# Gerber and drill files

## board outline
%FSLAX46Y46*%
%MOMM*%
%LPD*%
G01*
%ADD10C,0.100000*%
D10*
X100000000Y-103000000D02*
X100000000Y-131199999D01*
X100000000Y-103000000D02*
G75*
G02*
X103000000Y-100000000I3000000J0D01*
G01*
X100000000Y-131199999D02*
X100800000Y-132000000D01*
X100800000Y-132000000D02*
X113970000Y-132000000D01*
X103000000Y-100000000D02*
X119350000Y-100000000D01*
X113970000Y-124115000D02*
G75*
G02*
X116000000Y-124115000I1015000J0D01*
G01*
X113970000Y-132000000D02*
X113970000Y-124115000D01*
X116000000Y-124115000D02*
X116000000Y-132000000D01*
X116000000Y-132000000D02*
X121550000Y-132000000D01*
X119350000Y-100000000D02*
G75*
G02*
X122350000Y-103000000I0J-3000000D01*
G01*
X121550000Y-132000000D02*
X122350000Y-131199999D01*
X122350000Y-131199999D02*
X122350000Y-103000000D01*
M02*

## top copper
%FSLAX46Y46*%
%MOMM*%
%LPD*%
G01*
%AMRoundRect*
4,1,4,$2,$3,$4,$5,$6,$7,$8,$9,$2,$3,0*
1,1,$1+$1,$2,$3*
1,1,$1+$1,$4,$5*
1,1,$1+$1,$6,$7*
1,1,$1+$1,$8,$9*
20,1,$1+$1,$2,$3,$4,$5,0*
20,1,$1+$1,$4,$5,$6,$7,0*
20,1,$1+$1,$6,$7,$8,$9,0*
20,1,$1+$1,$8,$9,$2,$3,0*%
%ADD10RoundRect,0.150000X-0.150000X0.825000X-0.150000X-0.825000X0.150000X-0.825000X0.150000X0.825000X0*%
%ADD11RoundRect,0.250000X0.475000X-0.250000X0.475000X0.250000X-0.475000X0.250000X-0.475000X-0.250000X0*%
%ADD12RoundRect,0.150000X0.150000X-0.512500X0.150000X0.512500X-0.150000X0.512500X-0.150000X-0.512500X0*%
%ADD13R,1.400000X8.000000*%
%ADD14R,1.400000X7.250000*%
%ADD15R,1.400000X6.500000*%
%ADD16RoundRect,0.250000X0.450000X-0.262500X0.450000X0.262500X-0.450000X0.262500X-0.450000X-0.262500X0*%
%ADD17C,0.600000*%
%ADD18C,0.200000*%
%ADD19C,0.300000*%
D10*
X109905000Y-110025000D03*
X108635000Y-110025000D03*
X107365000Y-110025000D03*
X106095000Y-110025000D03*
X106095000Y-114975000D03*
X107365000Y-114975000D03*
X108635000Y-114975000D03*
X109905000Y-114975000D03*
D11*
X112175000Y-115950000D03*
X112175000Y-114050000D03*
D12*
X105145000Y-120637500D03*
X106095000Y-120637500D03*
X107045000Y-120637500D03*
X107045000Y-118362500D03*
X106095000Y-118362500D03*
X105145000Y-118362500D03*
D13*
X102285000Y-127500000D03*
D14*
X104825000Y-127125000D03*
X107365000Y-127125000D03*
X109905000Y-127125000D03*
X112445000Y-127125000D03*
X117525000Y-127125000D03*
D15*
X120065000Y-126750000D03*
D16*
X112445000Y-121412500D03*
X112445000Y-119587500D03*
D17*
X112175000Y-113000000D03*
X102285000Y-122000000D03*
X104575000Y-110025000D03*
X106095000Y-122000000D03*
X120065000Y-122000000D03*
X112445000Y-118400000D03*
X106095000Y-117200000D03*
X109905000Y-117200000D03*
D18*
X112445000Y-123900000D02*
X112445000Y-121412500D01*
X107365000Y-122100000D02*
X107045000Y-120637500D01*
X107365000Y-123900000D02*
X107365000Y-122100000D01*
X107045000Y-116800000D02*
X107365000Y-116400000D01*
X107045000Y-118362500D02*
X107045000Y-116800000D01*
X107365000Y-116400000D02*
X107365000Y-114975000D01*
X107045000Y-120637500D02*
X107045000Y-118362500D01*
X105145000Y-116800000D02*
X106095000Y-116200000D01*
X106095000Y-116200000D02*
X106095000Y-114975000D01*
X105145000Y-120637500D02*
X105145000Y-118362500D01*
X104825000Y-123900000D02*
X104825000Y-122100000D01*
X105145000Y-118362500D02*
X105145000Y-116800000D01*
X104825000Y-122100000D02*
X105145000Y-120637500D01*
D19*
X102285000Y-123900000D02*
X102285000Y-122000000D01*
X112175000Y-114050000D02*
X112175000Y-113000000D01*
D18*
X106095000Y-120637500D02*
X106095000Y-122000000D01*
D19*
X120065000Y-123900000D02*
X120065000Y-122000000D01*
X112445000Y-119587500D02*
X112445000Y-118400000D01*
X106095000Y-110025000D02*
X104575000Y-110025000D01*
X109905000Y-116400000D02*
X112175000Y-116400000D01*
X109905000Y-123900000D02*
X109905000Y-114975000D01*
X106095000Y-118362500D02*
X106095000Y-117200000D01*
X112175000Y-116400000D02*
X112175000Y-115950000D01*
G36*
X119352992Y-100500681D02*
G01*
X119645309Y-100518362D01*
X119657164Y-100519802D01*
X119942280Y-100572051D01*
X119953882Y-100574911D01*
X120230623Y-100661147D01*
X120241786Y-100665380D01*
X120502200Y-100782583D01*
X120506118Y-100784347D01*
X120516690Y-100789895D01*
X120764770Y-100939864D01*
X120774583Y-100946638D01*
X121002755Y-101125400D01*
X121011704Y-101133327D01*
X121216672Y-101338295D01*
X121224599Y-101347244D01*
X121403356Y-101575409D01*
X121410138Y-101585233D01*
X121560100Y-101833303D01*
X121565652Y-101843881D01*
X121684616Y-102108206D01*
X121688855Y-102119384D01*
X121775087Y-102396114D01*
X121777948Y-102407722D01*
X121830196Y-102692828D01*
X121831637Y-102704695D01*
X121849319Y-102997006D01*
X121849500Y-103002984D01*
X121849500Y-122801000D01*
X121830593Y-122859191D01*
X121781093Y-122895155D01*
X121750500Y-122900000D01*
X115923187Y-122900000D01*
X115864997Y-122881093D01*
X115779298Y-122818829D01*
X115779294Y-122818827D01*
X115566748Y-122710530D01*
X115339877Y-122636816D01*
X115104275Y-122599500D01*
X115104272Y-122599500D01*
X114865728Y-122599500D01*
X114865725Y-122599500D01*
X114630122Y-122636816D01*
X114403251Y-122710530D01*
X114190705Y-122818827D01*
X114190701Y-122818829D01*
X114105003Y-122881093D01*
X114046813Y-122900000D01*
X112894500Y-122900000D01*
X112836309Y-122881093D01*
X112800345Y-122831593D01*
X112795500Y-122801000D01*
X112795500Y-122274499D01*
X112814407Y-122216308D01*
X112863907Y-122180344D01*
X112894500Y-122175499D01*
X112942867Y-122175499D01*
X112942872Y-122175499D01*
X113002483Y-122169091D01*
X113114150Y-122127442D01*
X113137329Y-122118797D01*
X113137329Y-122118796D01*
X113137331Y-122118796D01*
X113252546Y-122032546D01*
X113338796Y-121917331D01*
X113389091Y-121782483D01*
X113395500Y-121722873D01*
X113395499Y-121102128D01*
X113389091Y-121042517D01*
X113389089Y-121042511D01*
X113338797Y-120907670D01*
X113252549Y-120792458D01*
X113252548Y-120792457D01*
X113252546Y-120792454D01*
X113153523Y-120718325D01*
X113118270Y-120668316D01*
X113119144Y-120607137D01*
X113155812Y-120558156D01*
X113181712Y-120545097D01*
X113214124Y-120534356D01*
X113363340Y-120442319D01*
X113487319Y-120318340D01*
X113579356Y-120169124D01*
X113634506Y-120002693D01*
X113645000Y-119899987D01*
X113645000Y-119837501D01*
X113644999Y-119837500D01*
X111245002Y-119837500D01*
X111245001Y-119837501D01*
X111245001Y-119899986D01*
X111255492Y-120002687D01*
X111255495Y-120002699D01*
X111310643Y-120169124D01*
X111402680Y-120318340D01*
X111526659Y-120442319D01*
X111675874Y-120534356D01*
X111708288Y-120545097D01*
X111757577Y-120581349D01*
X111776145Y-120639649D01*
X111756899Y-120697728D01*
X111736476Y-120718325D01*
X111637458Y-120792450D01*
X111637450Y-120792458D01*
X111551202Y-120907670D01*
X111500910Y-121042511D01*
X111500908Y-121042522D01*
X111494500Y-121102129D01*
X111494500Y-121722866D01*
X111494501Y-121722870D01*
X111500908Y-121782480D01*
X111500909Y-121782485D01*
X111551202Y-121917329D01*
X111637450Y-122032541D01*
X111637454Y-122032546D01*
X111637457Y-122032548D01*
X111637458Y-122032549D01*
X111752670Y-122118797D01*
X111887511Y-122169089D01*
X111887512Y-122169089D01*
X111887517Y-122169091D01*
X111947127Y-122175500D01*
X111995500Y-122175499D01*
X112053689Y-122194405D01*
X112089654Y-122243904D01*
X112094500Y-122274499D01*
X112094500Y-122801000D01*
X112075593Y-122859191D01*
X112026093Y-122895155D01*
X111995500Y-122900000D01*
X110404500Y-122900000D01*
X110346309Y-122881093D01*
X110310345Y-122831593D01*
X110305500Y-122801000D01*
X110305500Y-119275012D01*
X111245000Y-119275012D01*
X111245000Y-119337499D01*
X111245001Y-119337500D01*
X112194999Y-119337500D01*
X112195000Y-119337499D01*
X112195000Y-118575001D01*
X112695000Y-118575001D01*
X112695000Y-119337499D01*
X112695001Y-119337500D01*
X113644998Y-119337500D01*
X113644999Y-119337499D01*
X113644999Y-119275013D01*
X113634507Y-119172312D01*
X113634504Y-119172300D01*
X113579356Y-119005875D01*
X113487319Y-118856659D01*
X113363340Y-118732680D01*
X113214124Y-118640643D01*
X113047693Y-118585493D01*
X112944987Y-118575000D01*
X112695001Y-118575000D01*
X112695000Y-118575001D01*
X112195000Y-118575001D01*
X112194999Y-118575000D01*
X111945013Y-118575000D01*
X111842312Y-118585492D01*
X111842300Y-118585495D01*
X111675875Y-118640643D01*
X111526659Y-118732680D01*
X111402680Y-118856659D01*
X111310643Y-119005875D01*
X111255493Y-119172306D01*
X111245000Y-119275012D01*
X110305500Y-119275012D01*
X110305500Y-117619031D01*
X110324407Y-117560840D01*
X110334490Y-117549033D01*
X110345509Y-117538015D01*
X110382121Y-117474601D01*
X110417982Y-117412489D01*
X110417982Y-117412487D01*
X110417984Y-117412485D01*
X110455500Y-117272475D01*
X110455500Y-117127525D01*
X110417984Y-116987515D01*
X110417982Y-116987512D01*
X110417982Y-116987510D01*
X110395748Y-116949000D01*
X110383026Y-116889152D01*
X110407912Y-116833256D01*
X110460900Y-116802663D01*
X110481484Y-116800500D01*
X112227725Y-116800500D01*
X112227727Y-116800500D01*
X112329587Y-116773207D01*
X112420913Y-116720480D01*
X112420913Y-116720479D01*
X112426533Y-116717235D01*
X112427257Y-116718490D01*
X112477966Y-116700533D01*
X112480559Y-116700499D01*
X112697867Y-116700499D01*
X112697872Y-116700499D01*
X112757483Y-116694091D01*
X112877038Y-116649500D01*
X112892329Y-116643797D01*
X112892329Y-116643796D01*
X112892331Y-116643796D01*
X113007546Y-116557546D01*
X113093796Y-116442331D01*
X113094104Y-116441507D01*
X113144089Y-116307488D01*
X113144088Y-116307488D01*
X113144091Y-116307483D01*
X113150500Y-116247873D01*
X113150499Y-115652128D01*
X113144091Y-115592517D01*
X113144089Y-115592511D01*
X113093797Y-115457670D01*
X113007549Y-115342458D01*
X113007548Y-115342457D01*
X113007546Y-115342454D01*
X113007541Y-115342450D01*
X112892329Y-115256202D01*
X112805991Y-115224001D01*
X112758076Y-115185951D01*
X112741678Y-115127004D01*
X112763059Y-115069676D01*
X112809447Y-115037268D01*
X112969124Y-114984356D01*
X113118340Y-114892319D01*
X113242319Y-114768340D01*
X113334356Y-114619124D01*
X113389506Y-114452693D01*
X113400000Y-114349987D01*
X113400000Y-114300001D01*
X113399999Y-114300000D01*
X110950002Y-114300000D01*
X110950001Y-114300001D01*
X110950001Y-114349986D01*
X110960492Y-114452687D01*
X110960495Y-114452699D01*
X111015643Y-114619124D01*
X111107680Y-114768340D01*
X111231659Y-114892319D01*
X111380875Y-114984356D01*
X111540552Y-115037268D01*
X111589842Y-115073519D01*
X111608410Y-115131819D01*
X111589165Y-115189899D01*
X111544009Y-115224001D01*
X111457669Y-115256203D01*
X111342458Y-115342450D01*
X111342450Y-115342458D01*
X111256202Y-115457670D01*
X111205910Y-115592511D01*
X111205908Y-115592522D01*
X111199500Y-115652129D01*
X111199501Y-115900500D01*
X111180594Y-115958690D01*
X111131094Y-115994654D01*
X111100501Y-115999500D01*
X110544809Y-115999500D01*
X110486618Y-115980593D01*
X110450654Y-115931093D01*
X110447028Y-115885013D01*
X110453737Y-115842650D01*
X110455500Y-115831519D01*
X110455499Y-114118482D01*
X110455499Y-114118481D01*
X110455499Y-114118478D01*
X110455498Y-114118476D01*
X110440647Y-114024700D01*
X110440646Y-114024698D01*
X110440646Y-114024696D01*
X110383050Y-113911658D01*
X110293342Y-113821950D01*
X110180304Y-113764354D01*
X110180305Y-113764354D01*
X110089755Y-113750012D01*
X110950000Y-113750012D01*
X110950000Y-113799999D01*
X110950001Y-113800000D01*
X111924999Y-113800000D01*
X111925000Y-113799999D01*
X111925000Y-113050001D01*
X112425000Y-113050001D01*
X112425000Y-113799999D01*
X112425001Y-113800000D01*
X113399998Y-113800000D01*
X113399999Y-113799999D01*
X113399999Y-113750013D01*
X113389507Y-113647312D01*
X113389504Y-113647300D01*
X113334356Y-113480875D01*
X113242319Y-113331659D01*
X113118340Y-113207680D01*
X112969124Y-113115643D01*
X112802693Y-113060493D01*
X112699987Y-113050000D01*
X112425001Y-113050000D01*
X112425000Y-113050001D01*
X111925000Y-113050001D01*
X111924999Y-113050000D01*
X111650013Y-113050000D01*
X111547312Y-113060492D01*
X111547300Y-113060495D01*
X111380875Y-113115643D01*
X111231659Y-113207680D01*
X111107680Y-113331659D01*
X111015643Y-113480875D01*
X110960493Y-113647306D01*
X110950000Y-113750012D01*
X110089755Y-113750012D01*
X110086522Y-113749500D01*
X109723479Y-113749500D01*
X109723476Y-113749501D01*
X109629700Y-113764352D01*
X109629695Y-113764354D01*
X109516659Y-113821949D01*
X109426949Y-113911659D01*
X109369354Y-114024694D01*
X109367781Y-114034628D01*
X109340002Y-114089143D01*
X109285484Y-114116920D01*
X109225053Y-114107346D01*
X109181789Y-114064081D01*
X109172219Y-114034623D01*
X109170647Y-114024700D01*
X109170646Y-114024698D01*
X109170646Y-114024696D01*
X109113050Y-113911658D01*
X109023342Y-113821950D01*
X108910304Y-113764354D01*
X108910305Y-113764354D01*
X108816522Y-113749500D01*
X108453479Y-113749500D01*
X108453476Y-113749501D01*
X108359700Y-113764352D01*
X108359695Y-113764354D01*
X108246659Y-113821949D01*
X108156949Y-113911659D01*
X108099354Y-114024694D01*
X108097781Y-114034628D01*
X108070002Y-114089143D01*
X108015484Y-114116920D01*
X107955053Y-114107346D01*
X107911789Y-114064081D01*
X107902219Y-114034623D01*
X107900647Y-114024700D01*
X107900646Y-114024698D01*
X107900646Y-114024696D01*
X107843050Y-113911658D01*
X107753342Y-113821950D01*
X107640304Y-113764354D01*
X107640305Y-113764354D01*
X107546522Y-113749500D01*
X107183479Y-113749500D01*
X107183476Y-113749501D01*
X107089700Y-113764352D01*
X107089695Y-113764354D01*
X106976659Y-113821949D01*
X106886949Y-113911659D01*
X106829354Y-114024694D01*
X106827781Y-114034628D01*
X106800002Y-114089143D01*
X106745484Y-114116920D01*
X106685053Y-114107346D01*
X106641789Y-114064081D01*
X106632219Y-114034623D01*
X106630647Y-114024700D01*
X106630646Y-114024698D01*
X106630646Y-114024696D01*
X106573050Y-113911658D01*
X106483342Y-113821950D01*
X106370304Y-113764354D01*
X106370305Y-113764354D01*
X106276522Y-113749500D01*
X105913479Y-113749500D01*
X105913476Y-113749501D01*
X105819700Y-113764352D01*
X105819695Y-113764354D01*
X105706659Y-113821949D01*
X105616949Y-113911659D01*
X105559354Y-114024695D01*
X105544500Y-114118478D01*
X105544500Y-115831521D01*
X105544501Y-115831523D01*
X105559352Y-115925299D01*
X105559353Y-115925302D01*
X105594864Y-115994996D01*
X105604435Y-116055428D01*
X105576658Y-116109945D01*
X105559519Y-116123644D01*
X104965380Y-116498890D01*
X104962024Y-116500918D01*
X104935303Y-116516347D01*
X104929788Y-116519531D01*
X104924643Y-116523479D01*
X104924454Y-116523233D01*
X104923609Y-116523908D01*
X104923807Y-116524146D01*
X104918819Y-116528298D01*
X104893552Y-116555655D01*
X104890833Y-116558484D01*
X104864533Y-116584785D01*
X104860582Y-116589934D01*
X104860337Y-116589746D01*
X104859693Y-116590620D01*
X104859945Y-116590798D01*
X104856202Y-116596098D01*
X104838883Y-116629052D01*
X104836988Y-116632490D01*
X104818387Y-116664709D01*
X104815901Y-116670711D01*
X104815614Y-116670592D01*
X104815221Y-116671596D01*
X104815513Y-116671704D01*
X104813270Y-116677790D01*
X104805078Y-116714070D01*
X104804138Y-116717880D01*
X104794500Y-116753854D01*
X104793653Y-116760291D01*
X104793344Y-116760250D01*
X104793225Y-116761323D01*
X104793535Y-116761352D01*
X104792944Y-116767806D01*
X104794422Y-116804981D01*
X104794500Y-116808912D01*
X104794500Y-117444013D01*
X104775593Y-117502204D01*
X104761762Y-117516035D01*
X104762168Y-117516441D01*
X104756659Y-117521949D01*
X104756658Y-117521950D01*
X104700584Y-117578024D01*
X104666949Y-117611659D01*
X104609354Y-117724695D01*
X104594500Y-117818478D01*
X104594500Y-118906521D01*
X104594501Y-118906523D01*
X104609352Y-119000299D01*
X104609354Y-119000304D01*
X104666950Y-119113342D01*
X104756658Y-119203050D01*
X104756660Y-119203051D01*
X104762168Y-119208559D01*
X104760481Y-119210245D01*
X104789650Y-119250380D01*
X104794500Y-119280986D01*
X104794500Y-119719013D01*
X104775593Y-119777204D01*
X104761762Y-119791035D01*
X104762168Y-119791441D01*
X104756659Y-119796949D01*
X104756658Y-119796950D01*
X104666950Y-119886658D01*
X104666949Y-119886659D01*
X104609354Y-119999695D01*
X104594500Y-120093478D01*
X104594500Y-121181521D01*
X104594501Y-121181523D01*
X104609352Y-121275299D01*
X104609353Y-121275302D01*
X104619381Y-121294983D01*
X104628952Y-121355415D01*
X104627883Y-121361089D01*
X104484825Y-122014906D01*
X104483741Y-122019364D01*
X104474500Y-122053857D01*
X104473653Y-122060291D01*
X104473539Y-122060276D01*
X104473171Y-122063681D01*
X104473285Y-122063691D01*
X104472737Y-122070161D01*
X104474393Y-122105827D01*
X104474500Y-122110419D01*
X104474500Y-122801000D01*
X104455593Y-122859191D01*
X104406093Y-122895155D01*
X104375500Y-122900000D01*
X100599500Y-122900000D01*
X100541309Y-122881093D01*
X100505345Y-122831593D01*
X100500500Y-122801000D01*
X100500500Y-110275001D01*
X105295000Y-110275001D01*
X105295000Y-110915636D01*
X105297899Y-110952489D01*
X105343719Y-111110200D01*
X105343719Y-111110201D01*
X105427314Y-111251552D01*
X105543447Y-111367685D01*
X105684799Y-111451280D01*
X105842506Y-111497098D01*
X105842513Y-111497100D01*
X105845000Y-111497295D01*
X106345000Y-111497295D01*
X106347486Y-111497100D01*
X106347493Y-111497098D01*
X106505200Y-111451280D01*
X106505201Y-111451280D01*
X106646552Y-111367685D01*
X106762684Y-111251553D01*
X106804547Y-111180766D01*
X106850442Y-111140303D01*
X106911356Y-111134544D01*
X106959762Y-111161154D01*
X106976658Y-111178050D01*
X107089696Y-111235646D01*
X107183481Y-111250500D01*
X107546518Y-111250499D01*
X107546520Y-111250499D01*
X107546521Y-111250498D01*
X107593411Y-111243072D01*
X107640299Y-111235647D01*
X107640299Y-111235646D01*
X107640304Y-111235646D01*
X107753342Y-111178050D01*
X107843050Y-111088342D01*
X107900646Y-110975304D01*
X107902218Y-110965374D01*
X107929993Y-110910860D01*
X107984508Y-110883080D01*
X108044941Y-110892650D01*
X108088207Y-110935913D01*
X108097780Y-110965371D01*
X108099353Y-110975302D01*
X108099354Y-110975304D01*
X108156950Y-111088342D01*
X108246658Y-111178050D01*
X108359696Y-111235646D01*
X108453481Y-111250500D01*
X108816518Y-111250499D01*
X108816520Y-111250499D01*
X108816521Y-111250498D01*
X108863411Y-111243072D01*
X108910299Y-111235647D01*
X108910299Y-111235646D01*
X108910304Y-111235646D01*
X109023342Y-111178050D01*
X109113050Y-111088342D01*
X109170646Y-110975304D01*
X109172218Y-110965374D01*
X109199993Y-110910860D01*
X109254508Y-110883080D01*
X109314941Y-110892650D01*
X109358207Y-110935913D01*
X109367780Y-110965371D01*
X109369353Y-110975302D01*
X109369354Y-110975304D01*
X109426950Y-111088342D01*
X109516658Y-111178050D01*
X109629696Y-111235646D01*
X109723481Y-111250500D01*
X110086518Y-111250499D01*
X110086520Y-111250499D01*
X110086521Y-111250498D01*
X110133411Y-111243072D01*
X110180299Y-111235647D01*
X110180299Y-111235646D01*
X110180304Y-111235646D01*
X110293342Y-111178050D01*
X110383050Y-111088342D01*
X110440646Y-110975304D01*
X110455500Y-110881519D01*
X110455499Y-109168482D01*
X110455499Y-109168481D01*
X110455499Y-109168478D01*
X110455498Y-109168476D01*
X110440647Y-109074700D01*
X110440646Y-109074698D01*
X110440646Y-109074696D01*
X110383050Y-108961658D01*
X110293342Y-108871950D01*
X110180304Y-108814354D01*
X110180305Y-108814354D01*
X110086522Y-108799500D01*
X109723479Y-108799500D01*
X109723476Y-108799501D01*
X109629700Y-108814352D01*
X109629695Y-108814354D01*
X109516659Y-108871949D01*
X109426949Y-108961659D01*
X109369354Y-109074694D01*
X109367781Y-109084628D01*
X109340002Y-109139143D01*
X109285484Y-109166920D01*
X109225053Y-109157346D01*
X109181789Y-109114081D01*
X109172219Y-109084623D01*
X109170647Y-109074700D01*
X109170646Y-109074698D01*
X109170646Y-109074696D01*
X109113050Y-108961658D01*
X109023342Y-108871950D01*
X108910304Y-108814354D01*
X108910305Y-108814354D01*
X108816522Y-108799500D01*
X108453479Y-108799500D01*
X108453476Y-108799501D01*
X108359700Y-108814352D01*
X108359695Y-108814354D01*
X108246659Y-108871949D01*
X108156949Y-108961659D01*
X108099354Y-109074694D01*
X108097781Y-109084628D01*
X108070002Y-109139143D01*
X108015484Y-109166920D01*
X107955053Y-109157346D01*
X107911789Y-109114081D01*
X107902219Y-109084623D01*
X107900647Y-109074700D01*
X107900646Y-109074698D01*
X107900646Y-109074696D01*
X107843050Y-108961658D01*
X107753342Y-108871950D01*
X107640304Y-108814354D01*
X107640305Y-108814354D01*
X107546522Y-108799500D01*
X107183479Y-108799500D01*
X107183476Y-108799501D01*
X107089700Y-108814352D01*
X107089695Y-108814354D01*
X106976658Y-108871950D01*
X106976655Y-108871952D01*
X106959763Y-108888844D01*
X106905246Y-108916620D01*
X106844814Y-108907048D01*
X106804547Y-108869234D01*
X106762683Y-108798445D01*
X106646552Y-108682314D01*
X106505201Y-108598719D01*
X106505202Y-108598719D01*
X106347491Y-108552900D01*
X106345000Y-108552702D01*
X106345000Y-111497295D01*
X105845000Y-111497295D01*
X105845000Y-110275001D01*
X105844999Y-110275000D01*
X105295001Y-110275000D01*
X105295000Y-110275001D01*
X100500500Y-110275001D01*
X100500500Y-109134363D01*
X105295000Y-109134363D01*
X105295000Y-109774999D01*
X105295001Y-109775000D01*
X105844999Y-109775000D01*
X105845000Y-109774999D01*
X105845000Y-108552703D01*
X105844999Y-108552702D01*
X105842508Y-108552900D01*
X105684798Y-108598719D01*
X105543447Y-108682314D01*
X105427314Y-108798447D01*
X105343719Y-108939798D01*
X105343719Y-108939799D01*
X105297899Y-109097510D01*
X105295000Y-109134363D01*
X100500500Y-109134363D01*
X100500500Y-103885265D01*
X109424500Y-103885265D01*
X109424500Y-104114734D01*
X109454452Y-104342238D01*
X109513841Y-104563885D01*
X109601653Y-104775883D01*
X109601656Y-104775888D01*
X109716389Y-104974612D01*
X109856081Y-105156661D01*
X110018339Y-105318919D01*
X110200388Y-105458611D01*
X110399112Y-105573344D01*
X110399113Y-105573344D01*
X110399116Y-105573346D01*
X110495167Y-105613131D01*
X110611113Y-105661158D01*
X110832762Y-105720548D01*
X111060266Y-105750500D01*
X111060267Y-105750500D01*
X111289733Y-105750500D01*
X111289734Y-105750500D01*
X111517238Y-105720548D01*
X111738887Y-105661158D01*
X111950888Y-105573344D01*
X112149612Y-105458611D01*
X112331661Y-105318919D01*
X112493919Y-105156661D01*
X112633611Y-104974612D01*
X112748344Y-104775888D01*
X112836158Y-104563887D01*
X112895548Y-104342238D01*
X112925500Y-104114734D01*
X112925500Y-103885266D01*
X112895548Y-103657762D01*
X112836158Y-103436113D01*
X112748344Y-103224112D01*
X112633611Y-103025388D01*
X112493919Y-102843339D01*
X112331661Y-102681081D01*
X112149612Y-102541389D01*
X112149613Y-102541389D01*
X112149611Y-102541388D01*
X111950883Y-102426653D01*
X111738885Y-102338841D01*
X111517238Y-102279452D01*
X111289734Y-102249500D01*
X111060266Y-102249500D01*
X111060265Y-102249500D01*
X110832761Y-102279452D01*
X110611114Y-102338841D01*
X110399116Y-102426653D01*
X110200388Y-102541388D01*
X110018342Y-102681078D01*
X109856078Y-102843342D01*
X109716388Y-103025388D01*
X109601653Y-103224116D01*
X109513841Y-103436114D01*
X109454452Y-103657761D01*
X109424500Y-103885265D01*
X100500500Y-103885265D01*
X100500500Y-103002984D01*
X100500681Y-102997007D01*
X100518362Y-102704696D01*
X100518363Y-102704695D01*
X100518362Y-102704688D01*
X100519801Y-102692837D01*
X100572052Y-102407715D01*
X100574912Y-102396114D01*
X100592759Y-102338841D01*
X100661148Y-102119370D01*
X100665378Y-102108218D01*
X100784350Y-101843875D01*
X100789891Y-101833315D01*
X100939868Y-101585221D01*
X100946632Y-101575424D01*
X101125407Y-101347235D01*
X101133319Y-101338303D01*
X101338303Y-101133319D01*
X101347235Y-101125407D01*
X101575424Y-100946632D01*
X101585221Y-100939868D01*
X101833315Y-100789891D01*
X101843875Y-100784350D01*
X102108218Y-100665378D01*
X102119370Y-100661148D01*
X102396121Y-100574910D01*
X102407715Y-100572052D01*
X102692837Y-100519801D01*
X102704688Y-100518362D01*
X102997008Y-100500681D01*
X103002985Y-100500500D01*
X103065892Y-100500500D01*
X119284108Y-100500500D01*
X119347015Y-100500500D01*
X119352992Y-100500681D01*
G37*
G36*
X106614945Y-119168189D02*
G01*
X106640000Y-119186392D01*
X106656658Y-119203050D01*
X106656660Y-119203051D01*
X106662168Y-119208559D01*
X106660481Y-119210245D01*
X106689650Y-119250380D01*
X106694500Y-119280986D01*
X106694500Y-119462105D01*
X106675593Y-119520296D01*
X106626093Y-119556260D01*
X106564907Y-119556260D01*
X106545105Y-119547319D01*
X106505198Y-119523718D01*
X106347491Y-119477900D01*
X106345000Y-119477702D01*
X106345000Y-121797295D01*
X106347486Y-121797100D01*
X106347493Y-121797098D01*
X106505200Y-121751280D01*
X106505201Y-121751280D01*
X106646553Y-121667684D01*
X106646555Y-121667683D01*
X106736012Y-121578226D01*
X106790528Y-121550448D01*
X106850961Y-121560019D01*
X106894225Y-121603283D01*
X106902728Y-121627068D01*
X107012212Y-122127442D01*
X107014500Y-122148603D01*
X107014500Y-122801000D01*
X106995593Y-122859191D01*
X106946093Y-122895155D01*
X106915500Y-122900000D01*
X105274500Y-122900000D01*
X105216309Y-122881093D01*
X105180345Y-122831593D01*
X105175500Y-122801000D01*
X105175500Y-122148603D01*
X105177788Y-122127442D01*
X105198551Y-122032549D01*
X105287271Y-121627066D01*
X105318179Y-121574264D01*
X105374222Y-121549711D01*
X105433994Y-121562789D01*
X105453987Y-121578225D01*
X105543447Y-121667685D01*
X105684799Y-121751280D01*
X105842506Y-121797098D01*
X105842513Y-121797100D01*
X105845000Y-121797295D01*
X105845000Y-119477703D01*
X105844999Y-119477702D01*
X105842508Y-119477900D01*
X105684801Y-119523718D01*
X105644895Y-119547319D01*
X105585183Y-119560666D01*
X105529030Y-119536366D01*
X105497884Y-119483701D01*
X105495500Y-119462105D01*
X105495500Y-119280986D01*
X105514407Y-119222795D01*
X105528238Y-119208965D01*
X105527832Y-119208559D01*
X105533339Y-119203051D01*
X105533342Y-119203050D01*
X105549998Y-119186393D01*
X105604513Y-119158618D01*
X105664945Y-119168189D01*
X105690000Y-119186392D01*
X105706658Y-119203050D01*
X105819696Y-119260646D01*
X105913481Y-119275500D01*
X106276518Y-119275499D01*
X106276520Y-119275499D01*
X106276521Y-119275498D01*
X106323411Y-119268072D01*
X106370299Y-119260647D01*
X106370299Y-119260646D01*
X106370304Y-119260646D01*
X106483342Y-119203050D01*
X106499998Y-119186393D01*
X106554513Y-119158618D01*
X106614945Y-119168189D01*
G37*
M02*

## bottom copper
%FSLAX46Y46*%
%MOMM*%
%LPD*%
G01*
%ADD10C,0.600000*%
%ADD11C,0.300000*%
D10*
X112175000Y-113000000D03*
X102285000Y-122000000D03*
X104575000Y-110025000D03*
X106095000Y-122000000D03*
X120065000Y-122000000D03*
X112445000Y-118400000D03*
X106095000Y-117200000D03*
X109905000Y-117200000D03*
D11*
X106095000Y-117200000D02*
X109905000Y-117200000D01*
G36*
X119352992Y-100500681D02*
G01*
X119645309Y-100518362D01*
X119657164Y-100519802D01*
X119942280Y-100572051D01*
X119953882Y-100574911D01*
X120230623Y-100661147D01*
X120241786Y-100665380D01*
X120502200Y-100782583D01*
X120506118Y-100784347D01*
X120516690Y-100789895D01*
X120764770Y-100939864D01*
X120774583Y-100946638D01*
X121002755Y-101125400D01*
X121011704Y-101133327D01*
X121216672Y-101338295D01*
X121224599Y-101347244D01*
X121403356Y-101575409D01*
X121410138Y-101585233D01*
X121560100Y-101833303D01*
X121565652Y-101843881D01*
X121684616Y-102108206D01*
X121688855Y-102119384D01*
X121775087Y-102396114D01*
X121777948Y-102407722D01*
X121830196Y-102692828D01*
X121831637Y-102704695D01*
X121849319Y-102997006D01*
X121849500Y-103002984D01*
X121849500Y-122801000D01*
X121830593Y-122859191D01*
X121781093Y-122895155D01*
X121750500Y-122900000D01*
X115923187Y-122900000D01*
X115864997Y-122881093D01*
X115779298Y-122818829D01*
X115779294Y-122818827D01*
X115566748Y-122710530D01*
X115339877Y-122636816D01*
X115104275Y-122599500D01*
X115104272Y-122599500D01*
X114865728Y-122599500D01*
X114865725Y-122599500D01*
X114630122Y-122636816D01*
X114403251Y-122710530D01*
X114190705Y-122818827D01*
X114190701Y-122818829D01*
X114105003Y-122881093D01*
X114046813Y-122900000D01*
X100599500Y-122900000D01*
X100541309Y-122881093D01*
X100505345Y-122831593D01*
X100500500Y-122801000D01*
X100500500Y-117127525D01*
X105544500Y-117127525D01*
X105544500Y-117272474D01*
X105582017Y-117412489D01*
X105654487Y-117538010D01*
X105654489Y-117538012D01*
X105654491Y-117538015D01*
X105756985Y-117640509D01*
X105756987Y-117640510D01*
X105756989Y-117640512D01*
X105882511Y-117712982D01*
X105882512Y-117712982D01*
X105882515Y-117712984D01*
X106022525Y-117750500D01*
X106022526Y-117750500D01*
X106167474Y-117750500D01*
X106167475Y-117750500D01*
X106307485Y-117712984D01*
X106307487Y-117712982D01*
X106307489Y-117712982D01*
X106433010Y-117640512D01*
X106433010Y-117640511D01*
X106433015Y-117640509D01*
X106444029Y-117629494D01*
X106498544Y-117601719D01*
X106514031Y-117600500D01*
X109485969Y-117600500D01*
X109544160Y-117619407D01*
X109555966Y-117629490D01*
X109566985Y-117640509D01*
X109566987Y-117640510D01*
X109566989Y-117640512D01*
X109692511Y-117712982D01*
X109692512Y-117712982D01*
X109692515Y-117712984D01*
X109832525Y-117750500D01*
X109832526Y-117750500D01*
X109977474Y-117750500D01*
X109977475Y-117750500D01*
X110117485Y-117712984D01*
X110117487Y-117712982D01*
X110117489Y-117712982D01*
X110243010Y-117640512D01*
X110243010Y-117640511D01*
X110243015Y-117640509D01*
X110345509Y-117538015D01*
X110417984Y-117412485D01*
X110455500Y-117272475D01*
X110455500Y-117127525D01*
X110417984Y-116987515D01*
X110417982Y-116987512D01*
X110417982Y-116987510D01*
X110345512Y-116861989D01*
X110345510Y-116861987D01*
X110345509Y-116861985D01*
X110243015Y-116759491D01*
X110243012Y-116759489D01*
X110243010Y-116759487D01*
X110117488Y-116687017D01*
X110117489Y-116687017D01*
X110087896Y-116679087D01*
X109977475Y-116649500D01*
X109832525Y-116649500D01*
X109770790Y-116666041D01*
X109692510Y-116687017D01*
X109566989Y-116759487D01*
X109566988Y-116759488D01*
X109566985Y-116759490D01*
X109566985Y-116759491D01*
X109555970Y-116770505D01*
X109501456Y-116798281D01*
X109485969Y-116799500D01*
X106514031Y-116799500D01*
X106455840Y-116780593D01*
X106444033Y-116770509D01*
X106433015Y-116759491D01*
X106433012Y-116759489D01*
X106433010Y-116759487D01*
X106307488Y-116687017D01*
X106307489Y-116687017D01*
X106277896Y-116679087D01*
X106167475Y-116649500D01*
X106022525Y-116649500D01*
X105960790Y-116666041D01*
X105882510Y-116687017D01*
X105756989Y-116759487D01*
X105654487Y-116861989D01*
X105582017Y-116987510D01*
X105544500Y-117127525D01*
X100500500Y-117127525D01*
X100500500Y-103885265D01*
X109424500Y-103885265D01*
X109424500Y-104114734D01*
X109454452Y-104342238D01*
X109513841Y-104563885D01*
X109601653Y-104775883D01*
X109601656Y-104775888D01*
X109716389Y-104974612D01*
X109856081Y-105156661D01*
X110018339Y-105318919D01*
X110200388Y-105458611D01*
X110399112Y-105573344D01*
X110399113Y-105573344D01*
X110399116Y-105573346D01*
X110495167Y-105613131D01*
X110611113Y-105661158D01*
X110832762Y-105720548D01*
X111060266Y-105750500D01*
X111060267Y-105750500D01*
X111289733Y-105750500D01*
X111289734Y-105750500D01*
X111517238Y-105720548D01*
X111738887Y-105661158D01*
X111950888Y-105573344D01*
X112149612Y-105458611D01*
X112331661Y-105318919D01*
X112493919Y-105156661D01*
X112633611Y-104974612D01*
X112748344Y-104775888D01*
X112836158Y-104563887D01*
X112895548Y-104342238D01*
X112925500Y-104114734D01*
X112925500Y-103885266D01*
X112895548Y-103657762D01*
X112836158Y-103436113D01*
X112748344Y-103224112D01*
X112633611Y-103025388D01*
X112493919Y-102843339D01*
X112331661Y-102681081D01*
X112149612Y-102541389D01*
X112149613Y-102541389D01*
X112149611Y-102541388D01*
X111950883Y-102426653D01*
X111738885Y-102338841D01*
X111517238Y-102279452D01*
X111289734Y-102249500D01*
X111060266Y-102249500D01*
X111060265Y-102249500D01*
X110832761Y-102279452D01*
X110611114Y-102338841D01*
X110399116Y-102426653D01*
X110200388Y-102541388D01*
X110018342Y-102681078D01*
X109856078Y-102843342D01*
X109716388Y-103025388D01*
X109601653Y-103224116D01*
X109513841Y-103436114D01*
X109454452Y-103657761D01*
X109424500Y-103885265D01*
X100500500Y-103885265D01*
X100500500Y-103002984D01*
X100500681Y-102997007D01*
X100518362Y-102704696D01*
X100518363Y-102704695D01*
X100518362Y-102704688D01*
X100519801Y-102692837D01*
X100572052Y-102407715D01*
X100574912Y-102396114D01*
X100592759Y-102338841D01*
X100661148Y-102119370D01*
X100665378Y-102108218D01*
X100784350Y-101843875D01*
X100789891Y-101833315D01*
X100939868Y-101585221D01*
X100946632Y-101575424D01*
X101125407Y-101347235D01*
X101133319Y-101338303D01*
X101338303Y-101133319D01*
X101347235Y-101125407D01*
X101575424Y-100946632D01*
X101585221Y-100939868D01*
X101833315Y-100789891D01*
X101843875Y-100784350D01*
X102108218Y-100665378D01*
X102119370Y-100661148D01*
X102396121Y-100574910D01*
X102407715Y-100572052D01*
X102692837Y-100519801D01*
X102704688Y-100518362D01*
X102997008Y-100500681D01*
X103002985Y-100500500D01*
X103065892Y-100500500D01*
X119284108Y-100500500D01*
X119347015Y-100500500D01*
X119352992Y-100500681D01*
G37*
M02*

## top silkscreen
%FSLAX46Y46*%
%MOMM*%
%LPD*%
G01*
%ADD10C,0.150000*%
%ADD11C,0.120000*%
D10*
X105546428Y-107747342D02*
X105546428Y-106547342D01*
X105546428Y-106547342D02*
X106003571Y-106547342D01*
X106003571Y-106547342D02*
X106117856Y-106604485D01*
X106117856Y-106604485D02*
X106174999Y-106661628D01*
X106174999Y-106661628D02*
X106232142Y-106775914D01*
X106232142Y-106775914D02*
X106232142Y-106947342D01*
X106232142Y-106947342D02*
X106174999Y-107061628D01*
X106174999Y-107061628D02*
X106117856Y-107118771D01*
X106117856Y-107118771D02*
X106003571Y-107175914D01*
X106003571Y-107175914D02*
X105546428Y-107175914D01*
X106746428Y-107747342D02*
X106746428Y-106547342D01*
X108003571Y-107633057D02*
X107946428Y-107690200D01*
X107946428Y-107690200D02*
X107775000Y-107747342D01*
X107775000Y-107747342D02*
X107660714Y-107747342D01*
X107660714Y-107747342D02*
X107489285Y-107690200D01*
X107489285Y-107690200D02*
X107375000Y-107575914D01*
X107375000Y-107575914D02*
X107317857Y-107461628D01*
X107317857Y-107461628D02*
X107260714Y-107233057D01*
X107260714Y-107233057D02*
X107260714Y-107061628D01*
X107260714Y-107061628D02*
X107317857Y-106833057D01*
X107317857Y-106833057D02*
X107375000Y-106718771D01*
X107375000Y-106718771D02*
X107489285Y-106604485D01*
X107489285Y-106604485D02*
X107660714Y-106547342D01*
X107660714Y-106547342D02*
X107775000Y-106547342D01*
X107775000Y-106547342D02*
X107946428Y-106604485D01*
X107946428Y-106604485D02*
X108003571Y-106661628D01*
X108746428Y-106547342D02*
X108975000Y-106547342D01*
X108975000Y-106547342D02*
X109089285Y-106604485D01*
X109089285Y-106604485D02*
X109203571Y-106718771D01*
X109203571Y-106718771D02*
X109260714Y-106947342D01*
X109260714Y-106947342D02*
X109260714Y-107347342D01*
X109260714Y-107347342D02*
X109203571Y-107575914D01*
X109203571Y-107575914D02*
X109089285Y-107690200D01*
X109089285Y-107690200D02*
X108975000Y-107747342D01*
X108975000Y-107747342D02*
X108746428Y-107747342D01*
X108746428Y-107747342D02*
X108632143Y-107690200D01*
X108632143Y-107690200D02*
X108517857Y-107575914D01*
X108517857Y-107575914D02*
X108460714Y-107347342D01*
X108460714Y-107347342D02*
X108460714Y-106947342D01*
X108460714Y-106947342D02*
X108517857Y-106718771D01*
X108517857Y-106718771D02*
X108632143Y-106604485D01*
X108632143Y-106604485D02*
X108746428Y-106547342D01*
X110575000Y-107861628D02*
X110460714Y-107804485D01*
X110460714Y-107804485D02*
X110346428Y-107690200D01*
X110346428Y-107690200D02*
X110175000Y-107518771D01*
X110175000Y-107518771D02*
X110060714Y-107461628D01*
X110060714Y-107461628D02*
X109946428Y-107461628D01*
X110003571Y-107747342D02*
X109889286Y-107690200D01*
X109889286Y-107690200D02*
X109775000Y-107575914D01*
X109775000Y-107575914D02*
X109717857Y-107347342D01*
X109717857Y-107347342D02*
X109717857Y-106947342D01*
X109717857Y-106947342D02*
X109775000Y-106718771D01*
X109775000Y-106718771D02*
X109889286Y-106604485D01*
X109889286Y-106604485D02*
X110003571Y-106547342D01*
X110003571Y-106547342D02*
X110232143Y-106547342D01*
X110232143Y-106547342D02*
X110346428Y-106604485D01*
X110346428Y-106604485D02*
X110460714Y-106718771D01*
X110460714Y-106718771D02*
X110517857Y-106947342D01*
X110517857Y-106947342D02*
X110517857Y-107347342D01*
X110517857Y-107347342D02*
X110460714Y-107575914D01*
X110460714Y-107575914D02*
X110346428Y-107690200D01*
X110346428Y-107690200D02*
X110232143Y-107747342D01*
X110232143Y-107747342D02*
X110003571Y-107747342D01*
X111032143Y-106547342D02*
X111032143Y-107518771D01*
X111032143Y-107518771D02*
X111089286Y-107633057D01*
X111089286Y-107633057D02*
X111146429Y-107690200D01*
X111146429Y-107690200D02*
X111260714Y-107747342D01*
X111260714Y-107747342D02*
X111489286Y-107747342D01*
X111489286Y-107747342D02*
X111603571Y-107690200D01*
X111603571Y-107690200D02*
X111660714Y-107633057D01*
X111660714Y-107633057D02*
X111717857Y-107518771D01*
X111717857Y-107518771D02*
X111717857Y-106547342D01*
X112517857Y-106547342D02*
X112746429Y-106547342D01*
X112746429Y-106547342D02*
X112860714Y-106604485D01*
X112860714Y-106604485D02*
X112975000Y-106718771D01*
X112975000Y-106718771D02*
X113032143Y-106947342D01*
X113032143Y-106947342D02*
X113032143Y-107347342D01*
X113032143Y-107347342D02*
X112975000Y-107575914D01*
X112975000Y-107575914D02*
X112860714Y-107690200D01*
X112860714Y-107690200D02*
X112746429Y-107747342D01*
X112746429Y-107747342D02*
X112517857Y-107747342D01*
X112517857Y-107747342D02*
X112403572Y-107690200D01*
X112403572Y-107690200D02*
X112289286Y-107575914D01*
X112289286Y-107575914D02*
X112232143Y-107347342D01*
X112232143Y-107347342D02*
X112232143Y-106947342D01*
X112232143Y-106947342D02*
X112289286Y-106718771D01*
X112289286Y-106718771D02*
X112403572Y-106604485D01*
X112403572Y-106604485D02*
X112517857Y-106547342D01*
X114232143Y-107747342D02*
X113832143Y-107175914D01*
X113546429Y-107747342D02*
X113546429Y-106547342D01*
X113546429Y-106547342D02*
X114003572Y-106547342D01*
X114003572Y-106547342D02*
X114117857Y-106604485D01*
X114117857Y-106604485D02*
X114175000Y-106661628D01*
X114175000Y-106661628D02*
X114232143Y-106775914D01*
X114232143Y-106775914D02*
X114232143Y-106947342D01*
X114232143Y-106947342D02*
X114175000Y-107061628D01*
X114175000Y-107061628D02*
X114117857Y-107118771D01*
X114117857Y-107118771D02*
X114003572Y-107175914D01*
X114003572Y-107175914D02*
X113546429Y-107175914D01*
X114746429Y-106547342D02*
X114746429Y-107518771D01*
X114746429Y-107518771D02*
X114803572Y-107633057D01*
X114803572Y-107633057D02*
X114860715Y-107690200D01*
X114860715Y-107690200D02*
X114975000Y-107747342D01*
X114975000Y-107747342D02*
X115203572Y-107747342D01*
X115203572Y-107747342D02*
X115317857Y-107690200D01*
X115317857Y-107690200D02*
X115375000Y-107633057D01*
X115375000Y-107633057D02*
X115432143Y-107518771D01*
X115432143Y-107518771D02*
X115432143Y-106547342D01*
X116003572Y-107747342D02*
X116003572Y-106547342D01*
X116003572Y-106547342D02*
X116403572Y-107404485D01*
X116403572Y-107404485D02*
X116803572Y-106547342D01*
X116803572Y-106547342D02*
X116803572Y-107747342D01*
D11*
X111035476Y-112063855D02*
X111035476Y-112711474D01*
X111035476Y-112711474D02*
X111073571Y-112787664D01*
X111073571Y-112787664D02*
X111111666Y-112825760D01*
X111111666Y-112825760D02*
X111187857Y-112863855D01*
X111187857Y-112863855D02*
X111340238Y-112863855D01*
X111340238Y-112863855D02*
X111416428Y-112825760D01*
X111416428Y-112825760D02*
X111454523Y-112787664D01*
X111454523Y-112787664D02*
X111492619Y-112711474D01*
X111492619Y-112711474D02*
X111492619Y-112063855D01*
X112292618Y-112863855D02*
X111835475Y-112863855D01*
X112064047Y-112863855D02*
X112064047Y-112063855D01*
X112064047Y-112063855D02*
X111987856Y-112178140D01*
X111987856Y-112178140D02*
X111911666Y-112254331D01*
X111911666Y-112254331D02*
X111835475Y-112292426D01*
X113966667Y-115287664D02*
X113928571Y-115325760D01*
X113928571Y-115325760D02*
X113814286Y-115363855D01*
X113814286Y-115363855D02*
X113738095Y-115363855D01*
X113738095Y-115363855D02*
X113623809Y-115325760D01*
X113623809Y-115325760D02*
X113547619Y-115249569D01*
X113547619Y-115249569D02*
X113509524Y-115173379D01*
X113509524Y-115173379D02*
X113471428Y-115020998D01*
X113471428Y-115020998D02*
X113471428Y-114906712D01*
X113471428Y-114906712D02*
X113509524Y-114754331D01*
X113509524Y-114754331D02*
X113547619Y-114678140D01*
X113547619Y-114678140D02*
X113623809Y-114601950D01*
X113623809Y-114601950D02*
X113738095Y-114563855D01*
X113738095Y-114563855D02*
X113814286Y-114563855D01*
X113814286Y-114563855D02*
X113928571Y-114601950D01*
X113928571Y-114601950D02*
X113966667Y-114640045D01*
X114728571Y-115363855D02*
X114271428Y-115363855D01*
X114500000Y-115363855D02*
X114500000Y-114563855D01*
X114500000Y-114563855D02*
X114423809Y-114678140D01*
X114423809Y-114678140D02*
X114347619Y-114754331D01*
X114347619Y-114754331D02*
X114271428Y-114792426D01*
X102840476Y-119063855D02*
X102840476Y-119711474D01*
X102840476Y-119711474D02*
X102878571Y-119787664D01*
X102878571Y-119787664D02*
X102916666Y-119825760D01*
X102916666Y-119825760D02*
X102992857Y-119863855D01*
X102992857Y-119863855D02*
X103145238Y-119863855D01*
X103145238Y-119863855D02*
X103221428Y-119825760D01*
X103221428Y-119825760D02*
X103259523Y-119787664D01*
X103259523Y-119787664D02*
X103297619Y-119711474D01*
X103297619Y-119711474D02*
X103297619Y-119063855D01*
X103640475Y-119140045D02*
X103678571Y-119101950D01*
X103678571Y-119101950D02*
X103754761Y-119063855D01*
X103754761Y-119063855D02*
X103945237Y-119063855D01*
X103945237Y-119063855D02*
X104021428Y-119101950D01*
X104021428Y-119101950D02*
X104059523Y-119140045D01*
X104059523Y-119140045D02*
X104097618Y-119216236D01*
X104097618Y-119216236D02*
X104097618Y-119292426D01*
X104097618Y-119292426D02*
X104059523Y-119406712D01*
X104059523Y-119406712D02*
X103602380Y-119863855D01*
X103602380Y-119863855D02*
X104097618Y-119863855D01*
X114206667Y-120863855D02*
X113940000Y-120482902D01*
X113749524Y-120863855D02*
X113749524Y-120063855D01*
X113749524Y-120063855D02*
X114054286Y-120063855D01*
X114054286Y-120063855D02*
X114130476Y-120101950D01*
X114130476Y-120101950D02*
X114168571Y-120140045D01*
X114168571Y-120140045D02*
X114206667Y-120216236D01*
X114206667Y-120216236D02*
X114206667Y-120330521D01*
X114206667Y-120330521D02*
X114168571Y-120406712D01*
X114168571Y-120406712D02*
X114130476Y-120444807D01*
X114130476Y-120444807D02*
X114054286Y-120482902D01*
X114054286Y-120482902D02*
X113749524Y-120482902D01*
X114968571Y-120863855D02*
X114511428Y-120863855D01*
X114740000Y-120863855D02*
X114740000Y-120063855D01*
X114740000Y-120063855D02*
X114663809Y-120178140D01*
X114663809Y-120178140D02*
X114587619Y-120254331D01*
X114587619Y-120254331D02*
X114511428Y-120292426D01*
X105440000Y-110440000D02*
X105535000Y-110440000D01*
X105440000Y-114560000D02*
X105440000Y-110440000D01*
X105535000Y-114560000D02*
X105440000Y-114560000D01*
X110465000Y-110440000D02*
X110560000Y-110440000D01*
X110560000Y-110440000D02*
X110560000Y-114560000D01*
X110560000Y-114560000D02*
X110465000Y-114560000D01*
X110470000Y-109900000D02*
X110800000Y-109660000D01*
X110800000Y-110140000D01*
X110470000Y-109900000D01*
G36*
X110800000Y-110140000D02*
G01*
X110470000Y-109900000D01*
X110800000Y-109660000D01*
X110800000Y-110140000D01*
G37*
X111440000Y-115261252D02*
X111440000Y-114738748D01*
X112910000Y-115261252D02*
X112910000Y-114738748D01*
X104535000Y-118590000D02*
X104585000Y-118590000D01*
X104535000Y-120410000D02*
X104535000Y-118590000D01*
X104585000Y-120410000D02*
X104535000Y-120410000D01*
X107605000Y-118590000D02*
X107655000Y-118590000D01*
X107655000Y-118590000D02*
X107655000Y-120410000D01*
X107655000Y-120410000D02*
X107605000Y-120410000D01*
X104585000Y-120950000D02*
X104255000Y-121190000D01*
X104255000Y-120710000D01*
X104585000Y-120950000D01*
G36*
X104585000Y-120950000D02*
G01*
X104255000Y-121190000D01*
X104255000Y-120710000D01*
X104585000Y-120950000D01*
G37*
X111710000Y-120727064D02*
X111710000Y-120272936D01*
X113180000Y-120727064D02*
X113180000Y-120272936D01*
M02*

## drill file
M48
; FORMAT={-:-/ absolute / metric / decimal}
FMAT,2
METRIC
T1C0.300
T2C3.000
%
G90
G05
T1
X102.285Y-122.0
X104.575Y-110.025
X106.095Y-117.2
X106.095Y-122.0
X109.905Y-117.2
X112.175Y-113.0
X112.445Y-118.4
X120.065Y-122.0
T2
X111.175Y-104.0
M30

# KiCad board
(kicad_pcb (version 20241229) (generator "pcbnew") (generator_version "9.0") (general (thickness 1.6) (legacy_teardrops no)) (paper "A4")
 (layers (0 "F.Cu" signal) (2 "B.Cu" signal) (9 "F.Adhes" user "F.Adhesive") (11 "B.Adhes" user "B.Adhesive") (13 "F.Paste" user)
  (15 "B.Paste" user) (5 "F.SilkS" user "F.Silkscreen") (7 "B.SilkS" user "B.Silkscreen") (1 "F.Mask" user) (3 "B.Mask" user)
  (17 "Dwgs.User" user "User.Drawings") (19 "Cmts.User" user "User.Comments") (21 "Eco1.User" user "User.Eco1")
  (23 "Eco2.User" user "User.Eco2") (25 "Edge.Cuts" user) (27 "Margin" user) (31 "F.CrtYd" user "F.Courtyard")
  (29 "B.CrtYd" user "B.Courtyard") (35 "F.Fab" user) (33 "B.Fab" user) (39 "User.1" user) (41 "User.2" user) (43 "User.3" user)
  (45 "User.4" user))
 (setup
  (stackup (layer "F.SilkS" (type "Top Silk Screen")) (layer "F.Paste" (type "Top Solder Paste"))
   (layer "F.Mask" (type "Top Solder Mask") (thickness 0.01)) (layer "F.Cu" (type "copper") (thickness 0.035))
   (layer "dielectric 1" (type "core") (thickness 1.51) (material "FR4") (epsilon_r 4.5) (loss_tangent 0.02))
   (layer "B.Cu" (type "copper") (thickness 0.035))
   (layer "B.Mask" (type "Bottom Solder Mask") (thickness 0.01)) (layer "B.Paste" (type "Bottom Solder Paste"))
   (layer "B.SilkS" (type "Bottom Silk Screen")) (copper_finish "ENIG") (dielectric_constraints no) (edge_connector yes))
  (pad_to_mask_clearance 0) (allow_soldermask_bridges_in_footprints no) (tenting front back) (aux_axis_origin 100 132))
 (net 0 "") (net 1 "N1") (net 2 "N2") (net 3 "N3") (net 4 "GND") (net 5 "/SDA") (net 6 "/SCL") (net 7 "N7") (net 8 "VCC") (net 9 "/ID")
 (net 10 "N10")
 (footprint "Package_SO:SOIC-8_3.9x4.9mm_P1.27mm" (layer "F.Cu") (at 108 112.5 -90)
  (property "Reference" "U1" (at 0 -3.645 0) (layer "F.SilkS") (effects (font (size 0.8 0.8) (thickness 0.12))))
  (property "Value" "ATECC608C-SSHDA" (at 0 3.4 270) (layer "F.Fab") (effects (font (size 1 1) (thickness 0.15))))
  (fp_line (start -2.06 2.56) (end -2.06 2.465) (stroke (width 0.12) (type solid)) (layer "F.SilkS"))
  (fp_line (start 2.06 2.56) (end -2.06 2.56) (stroke (width 0.12) (type solid)) (layer "F.SilkS"))
  (fp_line (start 2.06 2.465) (end 2.06 2.56) (stroke (width 0.12) (type solid)) (layer "F.SilkS"))
  (fp_line (start -2.06 -2.465) (end -2.06 -2.56) (stroke (width 0.12) (type solid)) (layer "F.SilkS"))
  (fp_line (start -2.06 -2.56) (end 2.06 -2.56) (stroke (width 0.12) (type solid)) (layer "F.SilkS"))
  (fp_line (start 2.06 -2.56) (end 2.06 -2.465) (stroke (width 0.12) (type solid)) (layer "F.SilkS"))
  (fp_poly (pts (xy -2.6 -2.47) (xy -2.84 -2.8) (xy -2.36 -2.8)) (stroke (width 0.12) (type solid)) (fill yes) (layer "F.SilkS"))
  (pad "1" smd roundrect (at -2.475 -1.905 270) (size 1.95 0.6) (layers "F.Cu" "F.Mask" "F.Paste") (roundrect_rratio 0.25) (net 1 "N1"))
  (pad "2" smd roundrect (at -2.475 -0.635 270) (size 1.95 0.6) (layers "F.Cu" "F.Mask" "F.Paste") (roundrect_rratio 0.25) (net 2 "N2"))
  (pad "3" smd roundrect (at -2.475 0.635 270) (size 1.95 0.6) (layers "F.Cu" "F.Mask" "F.Paste") (roundrect_rratio 0.25) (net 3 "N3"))
  (pad "4" smd roundrect (at -2.475 1.905 270) (size 1.95 0.6) (layers "F.Cu" "F.Mask" "F.Paste") (roundrect_rratio 0.25) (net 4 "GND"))
  (pad "5" smd roundrect (at 2.475 1.905 270) (size 1.95 0.6) (layers "F.Cu" "F.Mask" "F.Paste") (roundrect_rratio 0.25) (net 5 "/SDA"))
  (pad "6" smd roundrect (at 2.475 0.635 270) (size 1.95 0.6) (layers "F.Cu" "F.Mask" "F.Paste") (roundrect_rratio 0.25) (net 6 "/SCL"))
  (pad "7" smd roundrect (at 2.475 -0.635 270) (size 1.95 0.6) (layers "F.Cu" "F.Mask" "F.Paste") (roundrect_rratio 0.25) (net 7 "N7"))
  (pad "8" smd roundrect (at 2.475 -1.905 270) (size 1.95 0.6) (layers "F.Cu" "F.Mask" "F.Paste") (roundrect_rratio 0.25) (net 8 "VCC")))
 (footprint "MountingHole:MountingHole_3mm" (layer "F.Cu") (at 111.175 104)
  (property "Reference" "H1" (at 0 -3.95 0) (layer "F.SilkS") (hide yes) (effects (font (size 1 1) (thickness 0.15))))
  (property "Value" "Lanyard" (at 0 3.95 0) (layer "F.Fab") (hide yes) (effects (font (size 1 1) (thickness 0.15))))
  (pad "" np_thru_hole circle (at 0 0) (size 3 3) (drill 3) (layers "*.Cu" "*.Mask")))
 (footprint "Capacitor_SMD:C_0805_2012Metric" (layer "F.Cu") (at 112.175 115 90)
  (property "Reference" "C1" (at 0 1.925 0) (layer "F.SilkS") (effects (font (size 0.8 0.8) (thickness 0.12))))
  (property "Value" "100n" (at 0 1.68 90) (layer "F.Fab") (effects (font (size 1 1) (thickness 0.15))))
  (fp_line (start -0.261252 -0.735) (end 0.261252 -0.735) (stroke (width 0.12) (type solid)) (layer "F.SilkS"))
  (fp_line (start -0.261252 0.735) (end 0.261252 0.735) (stroke (width 0.12) (type solid)) (layer "F.SilkS"))
  (pad "1" smd roundrect (at -0.95 0 90) (size 1 1.45) (layers "F.Cu" "F.Mask" "F.Paste") (roundrect_rratio 0.25) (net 8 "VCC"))
  (pad "2" smd roundrect (at 0.95 0 90) (size 1 1.45) (layers "F.Cu" "F.Mask" "F.Paste") (roundrect_rratio 0.25) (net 4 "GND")))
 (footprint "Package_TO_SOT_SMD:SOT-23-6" (layer "F.Cu") (at 106.095 119.5 90)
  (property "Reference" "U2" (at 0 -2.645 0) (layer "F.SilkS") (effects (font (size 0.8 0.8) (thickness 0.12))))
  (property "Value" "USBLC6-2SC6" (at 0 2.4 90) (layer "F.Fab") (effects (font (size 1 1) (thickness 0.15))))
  (fp_line (start 0.91 -1.56) (end 0.91 -1.51) (stroke (width 0.12) (type solid)) (layer "F.SilkS"))
  (fp_line (start -0.91 -1.56) (end 0.91 -1.56) (stroke (width 0.12) (type solid)) (layer "F.SilkS"))
  (fp_line (start -0.91 -1.51) (end -0.91 -1.56) (stroke (width 0.12) (type solid)) (layer "F.SilkS"))
  (fp_line (start 0.91 1.51) (end 0.91 1.56) (stroke (width 0.12) (type solid)) (layer "F.SilkS"))
  (fp_line (start 0.91 1.56) (end -0.91 1.56) (stroke (width 0.12) (type solid)) (layer "F.SilkS"))
  (fp_line (start -0.91 1.56) (end -0.91 1.51) (stroke (width 0.12) (type solid)) (layer "F.SilkS"))
  (fp_poly (pts (xy -1.45 -1.51) (xy -1.69 -1.84) (xy -1.21 -1.84)) (stroke (width 0.12) (type solid)) (fill yes) (layer "F.SilkS"))
  (pad "1" smd roundrect (at -1.1375 -0.95 90) (size 1.325 0.6) (layers "F.Cu" "F.Mask" "F.Paste") (roundrect_rratio 0.25) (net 5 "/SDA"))
  (pad "2" smd roundrect (at -1.1375 0 90) (size 1.325 0.6) (layers "F.Cu" "F.Mask" "F.Paste") (roundrect_rratio 0.25) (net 4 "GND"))
  (pad "3" smd roundrect (at -1.1375 0.95 90) (size 1.325 0.6) (layers "F.Cu" "F.Mask" "F.Paste") (roundrect_rratio 0.25) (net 6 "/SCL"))
  (pad "4" smd roundrect (at 1.1375 0.95 90) (size 1.325 0.6) (layers "F.Cu" "F.Mask" "F.Paste") (roundrect_rratio 0.25) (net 6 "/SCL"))
  (pad "5" smd roundrect (at 1.1375 0 90) (size 1.325 0.6) (layers "F.Cu" "F.Mask" "F.Paste") (roundrect_rratio 0.25) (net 8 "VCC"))
  (pad "6" smd roundrect (at 1.1375 -0.95 90) (size 1.325 0.6) (layers "F.Cu" "F.Mask" "F.Paste") (roundrect_rratio 0.25) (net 5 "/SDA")))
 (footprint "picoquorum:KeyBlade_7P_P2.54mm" (layer "F.Cu") (at 111.175 132)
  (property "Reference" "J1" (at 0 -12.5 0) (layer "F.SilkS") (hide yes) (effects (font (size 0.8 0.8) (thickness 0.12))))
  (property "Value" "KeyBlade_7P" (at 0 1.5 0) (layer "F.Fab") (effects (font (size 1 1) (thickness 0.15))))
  (pad "1" smd rect (at -8.89 -4.5) (size 1.4 8) (layers "F.Cu" "F.Mask") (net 4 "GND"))
  (pad "2" smd rect (at -6.35 -4.875) (size 1.4 7.25) (layers "F.Cu" "F.Mask") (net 5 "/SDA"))
  (pad "3" smd rect (at -3.81 -4.875) (size 1.4 7.25) (layers "F.Cu" "F.Mask") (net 6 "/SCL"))
  (pad "4" smd rect (at -1.27 -4.875) (size 1.4 7.25) (layers "F.Cu" "F.Mask") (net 8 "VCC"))
  (pad "5" smd rect (at 1.27 -4.875) (size 1.4 7.25) (layers "F.Cu" "F.Mask") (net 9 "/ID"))
  (pad "7" smd rect (at 6.35 -4.875) (size 1.4 7.25) (layers "F.Cu" "F.Mask") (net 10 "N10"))
  (pad "8" smd rect (at 8.89 -5.25) (size 1.4 6.5) (layers "F.Cu" "F.Mask") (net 4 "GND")))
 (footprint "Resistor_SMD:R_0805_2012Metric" (layer "F.Cu") (at 112.445 120.5 90)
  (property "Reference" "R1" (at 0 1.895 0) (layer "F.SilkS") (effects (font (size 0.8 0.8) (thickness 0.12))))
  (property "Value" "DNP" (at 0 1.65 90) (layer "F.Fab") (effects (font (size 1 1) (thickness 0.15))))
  (fp_line (start -0.227064 -0.735) (end 0.227064 -0.735) (stroke (width 0.12) (type solid)) (layer "F.SilkS"))
  (fp_line (start -0.227064 0.735) (end 0.227064 0.735) (stroke (width 0.12) (type solid)) (layer "F.SilkS"))
  (pad "1" smd roundrect (at -0.9125 0 90) (size 1.025 1.4) (layers "F.Cu" "F.Mask" "F.Paste") (roundrect_rratio 0.243902) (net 9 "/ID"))
  (pad "2" smd roundrect (at 0.9125 0 90) (size 1.025 1.4) (layers "F.Cu" "F.Mask" "F.Paste") (roundrect_rratio 0.243902) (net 4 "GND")))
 (gr_line (start 100 103) (end 100 131.199999) (stroke (width 0.1) (type default)) (layer "Edge.Cuts"))
 (gr_arc (start 100 103) (mid 100.87868 100.87868) (end 103 100) (stroke (width 0.1) (type default)) (layer "Edge.Cuts"))
 (gr_line (start 100 131.199999) (end 100.8 132) (stroke (width 0.1) (type default)) (layer "Edge.Cuts"))
 (gr_line (start 100.8 132) (end 113.97 132) (stroke (width 0.1) (type default)) (layer "Edge.Cuts"))
 (gr_line (start 103 100) (end 119.35 100) (stroke (width 0.1) (type default)) (layer "Edge.Cuts"))
 (gr_arc (start 113.97 124.115) (mid 114.985 123.1) (end 116 124.115) (stroke (width 0.1) (type default)) (layer "Edge.Cuts"))
 (gr_line (start 113.97 132) (end 113.97 124.115) (stroke (width 0.1) (type default)) (layer "Edge.Cuts"))
 (gr_line (start 116 124.115) (end 116 132) (stroke (width 0.1) (type default)) (layer "Edge.Cuts"))
 (gr_line (start 116 132) (end 121.55 132) (stroke (width 0.1) (type default)) (layer "Edge.Cuts"))
 (gr_arc (start 119.35 100) (mid 121.47132 100.87868) (end 122.35 103) (stroke (width 0.1) (type default)) (layer "Edge.Cuts"))
 (gr_line (start 121.55 132) (end 122.35 131.199999) (stroke (width 0.1) (type default)) (layer "Edge.Cuts"))
 (gr_line (start 122.35 131.199999) (end 122.35 103) (stroke (width 0.1) (type default)) (layer "Edge.Cuts"))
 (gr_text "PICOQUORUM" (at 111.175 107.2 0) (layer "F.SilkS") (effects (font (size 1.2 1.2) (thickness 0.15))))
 (segment (start 112.445 123.9) (end 112.445 121.4125) (width 0.2) (layer "F.Cu") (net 9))
 (segment (start 107.365 122.1) (end 107.045 120.6375) (width 0.2) (layer "F.Cu") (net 6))
 (segment (start 107.365 123.9) (end 107.365 122.1) (width 0.2) (layer "F.Cu") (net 6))
 (segment (start 107.045 116.8) (end 107.365 116.4) (width 0.2) (layer "F.Cu") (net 6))
 (segment (start 107.045 118.3625) (end 107.045 116.8) (width 0.2) (layer "F.Cu") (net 6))
 (segment (start 107.365 116.4) (end 107.365 114.975) (width 0.2) (layer "F.Cu") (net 6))
 (segment (start 107.045 120.6375) (end 107.045 118.3625) (width 0.2) (layer "F.Cu") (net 6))
 (segment (start 105.145 116.8) (end 106.095 116.2) (width 0.2) (layer "F.Cu") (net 5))
 (segment (start 106.095 116.2) (end 106.095 114.975) (width 0.2) (layer "F.Cu") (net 5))
 (segment (start 105.145 120.6375) (end 105.145 118.3625) (width 0.2) (layer "F.Cu") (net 5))
 (segment (start 104.825 123.9) (end 104.825 122.1) (width 0.2) (layer "F.Cu") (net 5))
 (segment (start 105.145 118.3625) (end 105.145 116.8) (width 0.2) (layer "F.Cu") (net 5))
 (segment (start 104.825 122.1) (end 105.145 120.6375) (width 0.2) (layer "F.Cu") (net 5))
 (segment (start 102.285 123.9) (end 102.285 122) (width 0.3) (layer "F.Cu") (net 4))
 (segment (start 112.175 114.05) (end 112.175 113) (width 0.3) (layer "F.Cu") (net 4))
 (segment (start 106.095 120.6375) (end 106.095 122) (width 0.2) (layer "F.Cu") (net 4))
 (segment (start 120.065 123.9) (end 120.065 122) (width 0.3) (layer "F.Cu") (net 4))
 (segment (start 112.445 119.5875) (end 112.445 118.4) (width 0.3) (layer "F.Cu") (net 4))
 (segment (start 106.095 110.025) (end 104.575 110.025) (width 0.3) (layer "F.Cu") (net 4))
 (via (at 112.175 113) (size 0.6) (drill 0.3) (layers "F.Cu" "B.Cu") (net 4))
 (via (at 102.285 122) (size 0.6) (drill 0.3) (layers "F.Cu" "B.Cu") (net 4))
 (via (at 104.575 110.025) (size 0.6) (drill 0.3) (layers "F.Cu" "B.Cu") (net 4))
 (via (at 106.095 122) (size 0.6) (drill 0.3) (layers "F.Cu" "B.Cu") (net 4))
 (via (at 120.065 122) (size 0.6) (drill 0.3) (layers "F.Cu" "B.Cu") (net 4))
 (via (at 112.445 118.4) (size 0.6) (drill 0.3) (layers "F.Cu" "B.Cu") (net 4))
 (segment (start 109.905 116.4) (end 112.175 116.4) (width 0.3) (layer "F.Cu") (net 8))
 (segment (start 109.905 123.9) (end 109.905 114.975) (width 0.3) (layer "F.Cu") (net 8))
 (segment (start 106.095 118.3625) (end 106.095 117.2) (width 0.3) (layer "F.Cu") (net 8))
 (segment (start 112.175 116.4) (end 112.175 115.95) (width 0.3) (layer "F.Cu") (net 8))
 (via (at 106.095 117.2) (size 0.6) (drill 0.3) (layers "F.Cu" "B.Cu") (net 8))
 (via (at 109.905 117.2) (size 0.6) (drill 0.3) (layers "F.Cu" "B.Cu") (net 8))
 (segment (start 106.095 117.2) (end 109.905 117.2) (width 0.3) (layer "B.Cu") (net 8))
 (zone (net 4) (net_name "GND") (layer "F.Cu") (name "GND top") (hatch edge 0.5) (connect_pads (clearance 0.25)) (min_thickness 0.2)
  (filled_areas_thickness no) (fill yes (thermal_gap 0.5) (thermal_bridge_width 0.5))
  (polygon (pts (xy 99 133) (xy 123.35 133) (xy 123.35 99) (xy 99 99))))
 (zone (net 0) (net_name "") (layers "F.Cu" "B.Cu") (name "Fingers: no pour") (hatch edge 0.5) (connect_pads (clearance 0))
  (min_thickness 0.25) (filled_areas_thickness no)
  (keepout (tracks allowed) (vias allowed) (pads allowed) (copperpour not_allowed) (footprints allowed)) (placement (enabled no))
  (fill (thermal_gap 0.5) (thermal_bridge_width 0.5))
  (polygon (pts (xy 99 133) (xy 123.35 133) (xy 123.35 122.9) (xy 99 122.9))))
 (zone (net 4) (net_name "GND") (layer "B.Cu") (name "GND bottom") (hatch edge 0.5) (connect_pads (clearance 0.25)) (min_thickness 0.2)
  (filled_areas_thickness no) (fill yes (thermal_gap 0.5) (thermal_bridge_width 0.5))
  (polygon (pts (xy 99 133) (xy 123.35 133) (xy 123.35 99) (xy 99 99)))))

